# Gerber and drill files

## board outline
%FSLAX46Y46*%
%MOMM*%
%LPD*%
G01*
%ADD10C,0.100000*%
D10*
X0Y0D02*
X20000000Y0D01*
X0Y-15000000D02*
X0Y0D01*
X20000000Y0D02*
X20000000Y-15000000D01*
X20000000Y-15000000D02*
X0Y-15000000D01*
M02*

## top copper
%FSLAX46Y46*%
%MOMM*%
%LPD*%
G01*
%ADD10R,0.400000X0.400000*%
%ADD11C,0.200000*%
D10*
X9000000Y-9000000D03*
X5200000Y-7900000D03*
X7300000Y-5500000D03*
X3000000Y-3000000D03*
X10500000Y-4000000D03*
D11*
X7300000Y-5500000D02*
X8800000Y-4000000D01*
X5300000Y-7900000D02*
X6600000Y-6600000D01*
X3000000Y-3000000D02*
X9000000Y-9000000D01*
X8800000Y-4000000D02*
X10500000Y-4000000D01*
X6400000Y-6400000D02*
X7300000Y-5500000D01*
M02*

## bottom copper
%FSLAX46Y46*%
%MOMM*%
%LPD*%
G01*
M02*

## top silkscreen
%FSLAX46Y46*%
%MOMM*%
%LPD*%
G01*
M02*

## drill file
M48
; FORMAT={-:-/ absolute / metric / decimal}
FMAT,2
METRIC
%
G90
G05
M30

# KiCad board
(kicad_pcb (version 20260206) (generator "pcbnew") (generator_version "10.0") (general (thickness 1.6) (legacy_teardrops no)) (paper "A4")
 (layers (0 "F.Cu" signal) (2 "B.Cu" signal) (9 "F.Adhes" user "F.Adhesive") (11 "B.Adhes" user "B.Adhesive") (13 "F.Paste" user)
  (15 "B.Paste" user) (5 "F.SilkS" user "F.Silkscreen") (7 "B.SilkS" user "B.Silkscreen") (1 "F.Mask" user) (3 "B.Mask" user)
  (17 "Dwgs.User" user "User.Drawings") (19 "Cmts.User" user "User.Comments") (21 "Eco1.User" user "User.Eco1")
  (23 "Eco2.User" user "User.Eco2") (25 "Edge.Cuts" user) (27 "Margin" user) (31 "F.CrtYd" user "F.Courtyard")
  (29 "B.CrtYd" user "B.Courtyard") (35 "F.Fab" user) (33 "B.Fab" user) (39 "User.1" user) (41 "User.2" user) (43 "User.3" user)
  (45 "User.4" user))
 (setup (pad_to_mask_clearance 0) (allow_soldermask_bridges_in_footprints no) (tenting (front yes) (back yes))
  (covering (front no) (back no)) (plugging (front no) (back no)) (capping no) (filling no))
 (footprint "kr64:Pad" (layer "F.Cu") (at 9 9)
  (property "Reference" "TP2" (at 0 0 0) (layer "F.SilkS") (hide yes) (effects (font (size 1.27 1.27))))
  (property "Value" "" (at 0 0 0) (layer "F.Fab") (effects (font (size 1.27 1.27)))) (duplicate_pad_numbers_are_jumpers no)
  (pad "1" smd rect (at 0 0) (size 0.4 0.4) (layers "F.Cu" "F.Mask" "F.Paste") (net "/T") (thermal_bridge_angle 45)))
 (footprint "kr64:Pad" (layer "F.Cu") (at 5.2 7.9)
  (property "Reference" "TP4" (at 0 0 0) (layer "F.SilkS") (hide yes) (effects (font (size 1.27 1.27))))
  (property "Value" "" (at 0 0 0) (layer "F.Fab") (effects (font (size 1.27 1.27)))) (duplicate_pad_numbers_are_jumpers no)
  (pad "1" smd rect (at 0 0) (size 0.4 0.4) (layers "F.Cu" "F.Mask" "F.Paste") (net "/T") (thermal_bridge_angle 45)))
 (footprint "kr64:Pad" (layer "F.Cu") (at 7.3 5.5)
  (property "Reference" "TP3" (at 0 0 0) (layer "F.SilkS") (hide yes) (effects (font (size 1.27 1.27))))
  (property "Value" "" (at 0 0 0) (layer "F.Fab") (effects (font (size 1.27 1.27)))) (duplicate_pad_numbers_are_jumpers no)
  (pad "1" smd rect (at 0 0) (size 0.4 0.4) (layers "F.Cu" "F.Mask" "F.Paste") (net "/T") (thermal_bridge_angle 45)))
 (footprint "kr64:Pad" (layer "F.Cu") (at 3 3)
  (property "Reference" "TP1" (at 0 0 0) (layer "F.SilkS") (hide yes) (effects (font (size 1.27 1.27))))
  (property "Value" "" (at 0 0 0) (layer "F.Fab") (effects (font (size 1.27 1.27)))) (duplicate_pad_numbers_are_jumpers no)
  (pad "1" smd rect (at 0 0) (size 0.4 0.4) (layers "F.Cu" "F.Mask" "F.Paste") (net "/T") (thermal_bridge_angle 45)))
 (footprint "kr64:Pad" (layer "F.Cu") (at 10.5 4)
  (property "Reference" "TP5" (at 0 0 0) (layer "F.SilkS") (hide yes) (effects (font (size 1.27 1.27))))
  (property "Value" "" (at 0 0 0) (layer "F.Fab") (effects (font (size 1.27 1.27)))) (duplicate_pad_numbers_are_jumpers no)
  (pad "1" smd rect (at 0 0) (size 0.4 0.4) (layers "F.Cu" "F.Mask" "F.Paste") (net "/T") (thermal_bridge_angle 45)))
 (gr_line (start 0 0) (end 20 0) (stroke (width 0.1) (type default)) (layer "Edge.Cuts"))
 (gr_line (start 0 15) (end 0 0) (stroke (width 0.1) (type default)) (layer "Edge.Cuts"))
 (gr_line (start 20 0) (end 20 15) (stroke (width 0.1) (type default)) (layer "Edge.Cuts"))
 (gr_line (start 20 15) (end 0 15) (stroke (width 0.1) (type default)) (layer "Edge.Cuts"))
 (segment (start 7.3 5.5) (end 8.8 4) (width 0.2) (layer "F.Cu") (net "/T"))
 (segment (start 5.3 7.9) (end 6.6 6.6) (width 0.2) (layer "F.Cu") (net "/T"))
 (segment (start 3 3) (end 9 9) (width 0.2) (layer "F.Cu") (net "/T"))
 (segment (start 8.8 4) (end 10.5 4) (width 0.2) (layer "F.Cu") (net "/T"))
 (segment (start 6.4 6.4) (end 7.3 5.5) (width 0.2) (layer "F.Cu") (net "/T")))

